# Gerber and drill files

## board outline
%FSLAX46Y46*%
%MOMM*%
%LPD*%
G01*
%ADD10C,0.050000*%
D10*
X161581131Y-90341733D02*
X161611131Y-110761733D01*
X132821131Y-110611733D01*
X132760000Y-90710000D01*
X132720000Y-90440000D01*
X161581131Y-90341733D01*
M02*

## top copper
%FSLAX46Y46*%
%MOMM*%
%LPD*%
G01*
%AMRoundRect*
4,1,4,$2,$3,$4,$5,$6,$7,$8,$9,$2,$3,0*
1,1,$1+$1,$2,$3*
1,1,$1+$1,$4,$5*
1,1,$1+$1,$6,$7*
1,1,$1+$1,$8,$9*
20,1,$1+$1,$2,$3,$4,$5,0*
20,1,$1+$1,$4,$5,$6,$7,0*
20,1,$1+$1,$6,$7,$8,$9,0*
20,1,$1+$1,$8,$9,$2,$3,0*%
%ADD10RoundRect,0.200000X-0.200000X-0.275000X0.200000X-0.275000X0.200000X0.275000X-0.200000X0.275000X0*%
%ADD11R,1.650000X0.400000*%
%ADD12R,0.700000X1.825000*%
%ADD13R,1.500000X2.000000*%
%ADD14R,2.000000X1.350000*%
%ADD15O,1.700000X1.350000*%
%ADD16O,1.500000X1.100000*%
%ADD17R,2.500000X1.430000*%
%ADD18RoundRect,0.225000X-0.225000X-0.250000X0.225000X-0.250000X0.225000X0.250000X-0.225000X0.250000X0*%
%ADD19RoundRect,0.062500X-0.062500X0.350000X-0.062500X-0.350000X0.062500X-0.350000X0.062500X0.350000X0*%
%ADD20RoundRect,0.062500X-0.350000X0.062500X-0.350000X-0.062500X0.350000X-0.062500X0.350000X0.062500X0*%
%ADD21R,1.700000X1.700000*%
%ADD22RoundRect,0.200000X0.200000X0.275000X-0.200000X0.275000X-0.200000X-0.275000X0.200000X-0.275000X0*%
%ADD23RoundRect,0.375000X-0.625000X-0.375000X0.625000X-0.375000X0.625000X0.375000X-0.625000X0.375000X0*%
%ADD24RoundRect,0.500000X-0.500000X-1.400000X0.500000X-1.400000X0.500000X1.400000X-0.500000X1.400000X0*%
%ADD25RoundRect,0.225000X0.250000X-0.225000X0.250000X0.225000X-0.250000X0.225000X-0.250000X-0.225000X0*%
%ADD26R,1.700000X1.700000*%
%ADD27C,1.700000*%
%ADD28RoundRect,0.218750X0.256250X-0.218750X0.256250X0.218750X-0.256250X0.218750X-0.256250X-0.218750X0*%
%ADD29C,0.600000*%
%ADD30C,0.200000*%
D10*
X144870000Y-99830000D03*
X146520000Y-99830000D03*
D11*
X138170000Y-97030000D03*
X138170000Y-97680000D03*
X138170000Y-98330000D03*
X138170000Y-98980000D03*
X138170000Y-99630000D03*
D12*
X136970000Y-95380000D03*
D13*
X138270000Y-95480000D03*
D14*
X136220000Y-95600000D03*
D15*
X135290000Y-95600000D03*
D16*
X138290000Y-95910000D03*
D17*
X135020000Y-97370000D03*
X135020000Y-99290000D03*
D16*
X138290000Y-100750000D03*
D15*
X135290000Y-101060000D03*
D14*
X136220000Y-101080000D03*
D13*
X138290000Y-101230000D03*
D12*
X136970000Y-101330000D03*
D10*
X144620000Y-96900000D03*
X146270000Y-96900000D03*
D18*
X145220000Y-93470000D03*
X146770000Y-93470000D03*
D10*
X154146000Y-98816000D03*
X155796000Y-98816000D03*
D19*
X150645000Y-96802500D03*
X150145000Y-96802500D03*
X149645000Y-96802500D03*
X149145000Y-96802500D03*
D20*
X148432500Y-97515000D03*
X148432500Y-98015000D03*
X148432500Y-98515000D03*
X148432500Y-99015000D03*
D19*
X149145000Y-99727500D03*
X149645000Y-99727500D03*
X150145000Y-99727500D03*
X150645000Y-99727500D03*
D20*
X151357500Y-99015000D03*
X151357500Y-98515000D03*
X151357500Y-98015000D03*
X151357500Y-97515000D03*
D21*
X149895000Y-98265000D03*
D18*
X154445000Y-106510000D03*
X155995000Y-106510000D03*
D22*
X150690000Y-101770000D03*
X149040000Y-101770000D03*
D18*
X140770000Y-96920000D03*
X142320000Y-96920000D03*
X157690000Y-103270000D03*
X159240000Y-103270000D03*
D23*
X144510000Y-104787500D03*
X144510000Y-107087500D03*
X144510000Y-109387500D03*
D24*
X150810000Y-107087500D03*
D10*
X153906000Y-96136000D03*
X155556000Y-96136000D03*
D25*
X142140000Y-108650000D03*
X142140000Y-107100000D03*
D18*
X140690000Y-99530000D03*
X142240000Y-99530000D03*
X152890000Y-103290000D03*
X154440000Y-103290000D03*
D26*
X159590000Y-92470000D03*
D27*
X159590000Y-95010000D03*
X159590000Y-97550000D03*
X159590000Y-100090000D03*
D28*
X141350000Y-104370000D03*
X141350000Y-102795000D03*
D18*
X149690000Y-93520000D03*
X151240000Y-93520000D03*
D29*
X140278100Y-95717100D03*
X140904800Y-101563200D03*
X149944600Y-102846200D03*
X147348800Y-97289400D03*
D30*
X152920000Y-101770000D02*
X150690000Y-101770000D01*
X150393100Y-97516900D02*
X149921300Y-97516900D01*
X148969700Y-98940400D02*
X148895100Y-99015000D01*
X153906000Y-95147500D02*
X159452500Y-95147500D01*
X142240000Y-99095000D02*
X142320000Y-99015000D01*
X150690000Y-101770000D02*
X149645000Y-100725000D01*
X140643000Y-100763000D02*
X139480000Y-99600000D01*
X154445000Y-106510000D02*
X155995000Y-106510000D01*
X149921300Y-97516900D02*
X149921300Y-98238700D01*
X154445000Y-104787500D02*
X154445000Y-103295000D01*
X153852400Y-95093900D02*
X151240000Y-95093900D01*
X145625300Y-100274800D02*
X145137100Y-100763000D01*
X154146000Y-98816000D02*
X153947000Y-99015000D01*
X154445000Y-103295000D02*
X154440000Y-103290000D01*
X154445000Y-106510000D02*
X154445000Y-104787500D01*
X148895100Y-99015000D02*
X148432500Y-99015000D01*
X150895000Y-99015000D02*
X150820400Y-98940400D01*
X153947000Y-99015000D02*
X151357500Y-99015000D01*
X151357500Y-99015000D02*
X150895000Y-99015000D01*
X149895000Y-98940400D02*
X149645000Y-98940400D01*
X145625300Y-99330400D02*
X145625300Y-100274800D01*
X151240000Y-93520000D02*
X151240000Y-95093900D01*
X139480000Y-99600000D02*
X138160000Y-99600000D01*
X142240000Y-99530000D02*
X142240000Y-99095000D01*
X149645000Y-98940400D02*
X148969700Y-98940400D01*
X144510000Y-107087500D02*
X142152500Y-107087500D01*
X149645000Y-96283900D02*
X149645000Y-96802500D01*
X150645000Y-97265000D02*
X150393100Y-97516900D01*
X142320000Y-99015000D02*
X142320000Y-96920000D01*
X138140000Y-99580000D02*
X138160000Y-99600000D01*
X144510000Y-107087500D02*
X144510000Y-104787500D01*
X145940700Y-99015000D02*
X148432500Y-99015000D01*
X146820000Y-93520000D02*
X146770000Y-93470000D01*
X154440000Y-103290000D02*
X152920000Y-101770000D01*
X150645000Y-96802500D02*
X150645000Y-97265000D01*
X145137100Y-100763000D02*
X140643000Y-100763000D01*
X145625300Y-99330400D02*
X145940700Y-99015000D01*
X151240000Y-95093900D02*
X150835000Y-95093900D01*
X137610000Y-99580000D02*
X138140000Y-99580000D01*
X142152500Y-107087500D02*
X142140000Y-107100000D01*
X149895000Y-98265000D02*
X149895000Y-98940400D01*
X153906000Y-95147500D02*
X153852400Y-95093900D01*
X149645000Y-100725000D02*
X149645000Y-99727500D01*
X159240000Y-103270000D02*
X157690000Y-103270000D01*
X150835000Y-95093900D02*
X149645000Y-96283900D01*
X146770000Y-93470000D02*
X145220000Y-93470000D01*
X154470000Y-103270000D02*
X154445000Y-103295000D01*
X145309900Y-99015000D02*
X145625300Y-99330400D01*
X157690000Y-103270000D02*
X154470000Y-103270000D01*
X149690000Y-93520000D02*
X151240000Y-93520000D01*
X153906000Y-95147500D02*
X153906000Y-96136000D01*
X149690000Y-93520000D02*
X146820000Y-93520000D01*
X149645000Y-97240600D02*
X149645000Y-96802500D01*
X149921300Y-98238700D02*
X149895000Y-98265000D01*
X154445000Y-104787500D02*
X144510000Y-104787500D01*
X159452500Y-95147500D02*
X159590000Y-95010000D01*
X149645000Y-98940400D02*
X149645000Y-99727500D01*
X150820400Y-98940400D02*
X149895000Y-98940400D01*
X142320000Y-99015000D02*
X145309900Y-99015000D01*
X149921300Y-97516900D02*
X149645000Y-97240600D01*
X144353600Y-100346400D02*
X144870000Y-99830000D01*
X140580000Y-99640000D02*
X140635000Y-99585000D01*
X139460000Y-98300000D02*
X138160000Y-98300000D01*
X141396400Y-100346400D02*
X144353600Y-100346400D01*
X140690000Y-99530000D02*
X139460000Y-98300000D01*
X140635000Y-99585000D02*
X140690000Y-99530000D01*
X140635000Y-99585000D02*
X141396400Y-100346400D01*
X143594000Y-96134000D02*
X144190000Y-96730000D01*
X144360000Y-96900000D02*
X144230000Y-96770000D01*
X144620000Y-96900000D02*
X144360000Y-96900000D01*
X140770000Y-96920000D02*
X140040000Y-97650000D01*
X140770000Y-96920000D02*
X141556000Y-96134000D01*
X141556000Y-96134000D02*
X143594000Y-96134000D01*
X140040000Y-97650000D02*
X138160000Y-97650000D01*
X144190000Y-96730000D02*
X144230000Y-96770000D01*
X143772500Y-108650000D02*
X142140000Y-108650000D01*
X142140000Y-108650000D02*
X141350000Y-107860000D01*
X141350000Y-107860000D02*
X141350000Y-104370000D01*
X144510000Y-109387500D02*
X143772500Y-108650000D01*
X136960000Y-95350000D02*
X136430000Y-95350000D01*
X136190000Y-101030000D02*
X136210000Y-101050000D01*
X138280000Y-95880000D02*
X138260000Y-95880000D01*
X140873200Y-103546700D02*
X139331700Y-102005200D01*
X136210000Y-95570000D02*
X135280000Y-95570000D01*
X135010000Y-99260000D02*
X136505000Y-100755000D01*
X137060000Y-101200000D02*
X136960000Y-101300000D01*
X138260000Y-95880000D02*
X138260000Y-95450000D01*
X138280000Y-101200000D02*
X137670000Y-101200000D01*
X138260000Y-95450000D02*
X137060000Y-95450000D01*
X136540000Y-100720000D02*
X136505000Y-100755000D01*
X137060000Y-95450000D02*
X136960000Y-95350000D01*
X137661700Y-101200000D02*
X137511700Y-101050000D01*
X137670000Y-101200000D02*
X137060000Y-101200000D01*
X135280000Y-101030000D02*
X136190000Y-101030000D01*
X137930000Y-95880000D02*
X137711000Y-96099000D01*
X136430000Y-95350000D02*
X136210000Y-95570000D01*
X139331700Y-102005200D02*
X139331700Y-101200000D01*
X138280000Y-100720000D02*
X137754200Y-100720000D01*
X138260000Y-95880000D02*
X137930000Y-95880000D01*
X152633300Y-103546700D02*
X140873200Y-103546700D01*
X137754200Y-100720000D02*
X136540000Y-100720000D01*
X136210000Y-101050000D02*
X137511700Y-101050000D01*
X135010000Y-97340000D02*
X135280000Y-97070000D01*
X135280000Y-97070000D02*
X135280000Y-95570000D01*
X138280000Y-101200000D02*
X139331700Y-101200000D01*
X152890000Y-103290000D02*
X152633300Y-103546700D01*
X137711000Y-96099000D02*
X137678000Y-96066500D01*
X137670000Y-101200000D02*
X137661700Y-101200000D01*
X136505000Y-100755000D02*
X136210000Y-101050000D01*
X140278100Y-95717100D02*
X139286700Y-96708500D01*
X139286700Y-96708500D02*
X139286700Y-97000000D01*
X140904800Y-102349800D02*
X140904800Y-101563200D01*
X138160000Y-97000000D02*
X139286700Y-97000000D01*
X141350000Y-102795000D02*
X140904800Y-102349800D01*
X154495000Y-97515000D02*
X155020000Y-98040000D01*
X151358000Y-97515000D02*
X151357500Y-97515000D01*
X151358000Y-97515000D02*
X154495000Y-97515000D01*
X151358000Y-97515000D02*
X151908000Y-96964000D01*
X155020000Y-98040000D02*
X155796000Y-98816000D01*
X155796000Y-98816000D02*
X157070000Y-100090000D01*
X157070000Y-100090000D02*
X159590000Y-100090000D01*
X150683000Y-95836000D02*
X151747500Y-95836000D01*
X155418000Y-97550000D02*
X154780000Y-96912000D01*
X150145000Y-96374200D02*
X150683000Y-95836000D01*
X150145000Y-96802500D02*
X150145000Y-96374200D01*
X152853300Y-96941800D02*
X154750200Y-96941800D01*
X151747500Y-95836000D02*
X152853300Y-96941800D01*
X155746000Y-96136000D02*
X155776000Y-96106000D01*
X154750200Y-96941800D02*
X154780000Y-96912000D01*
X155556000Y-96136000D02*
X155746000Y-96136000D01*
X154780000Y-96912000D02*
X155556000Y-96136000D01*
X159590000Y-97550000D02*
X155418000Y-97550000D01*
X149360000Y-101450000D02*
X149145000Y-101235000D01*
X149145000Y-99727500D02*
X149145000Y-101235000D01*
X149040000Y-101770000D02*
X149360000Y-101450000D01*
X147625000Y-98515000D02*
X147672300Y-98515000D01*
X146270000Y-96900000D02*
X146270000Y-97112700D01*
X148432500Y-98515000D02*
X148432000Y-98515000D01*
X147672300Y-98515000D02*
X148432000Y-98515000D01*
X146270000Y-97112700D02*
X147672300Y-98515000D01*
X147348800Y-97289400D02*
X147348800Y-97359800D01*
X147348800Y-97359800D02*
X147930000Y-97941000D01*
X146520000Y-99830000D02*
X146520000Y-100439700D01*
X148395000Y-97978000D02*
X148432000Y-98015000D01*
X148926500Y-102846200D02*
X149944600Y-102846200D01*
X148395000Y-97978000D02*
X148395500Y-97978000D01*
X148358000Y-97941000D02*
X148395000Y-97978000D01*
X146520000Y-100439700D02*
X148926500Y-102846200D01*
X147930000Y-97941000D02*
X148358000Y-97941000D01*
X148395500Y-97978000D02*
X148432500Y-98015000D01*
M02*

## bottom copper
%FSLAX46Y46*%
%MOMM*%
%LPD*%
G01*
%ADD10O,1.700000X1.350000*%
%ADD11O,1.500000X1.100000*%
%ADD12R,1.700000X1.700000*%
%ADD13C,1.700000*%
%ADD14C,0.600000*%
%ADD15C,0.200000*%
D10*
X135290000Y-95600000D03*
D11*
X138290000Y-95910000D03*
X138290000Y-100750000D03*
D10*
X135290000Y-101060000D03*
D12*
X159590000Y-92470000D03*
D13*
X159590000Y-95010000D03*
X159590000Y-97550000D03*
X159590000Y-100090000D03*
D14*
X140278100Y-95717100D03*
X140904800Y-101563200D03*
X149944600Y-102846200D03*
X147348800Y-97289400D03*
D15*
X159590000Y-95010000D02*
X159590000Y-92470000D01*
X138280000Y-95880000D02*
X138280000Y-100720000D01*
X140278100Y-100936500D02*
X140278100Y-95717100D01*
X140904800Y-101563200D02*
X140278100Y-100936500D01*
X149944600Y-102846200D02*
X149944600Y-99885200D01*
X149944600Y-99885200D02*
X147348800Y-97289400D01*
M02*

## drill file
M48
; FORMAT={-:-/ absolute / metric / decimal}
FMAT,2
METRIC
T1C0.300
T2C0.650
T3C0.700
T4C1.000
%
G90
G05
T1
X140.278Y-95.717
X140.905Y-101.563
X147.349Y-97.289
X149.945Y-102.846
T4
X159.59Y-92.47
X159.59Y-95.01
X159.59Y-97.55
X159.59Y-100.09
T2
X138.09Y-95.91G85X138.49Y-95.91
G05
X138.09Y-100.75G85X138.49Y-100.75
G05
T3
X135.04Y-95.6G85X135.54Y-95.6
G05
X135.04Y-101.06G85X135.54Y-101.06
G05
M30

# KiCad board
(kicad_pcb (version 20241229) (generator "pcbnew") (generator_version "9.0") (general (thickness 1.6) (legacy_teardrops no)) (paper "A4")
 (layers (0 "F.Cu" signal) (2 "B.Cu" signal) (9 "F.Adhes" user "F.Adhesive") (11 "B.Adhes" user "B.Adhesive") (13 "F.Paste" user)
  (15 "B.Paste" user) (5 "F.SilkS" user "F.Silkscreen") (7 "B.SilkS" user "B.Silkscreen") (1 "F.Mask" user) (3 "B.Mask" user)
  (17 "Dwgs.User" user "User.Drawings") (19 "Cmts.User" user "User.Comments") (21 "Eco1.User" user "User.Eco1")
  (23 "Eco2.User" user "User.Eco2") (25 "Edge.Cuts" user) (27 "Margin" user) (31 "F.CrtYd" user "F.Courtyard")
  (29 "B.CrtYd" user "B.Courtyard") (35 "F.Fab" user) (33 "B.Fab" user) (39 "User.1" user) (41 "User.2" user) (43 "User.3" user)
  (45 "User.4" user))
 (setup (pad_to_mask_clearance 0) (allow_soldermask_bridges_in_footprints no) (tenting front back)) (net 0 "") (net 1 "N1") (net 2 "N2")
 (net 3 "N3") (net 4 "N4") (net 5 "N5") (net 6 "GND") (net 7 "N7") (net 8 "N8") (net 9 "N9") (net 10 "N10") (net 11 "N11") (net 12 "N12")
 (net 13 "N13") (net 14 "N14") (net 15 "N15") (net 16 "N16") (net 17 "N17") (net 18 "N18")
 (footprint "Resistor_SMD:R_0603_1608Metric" (layer "F.Cu") (at 145.695 99.83)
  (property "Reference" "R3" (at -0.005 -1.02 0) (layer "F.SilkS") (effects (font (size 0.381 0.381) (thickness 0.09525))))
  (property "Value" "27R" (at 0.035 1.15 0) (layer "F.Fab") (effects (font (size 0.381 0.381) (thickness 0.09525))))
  (pad "1" smd roundrect (at -0.825 0) (size 0.8 0.95) (layers "F.Cu" "F.Mask" "F.Paste") (roundrect_rratio 0.25) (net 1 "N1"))
  (pad "2" smd roundrect (at 0.825 0) (size 0.8 0.95) (layers "F.Cu" "F.Mask" "F.Paste") (roundrect_rratio 0.25) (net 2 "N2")))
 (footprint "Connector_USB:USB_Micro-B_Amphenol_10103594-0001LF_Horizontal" (layer "F.Cu") (at 136.405 98.355 -90)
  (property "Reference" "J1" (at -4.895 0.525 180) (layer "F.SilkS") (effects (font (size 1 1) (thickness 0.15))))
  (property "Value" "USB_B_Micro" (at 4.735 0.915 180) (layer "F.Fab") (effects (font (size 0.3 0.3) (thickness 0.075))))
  (pad "1" smd rect (at -1.325 -1.765) (size 1.65 0.4) (layers "F.Cu" "F.Mask" "F.Paste") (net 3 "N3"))
  (pad "2" smd rect (at -0.675 -1.765) (size 1.65 0.4) (layers "F.Cu" "F.Mask" "F.Paste") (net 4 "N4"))
  (pad "3" smd rect (at -0.025 -1.765) (size 1.65 0.4) (layers "F.Cu" "F.Mask" "F.Paste") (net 1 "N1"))
  (pad "4" smd rect (at 0.625 -1.765) (size 1.65 0.4) (layers "F.Cu" "F.Mask" "F.Paste") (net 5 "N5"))
  (pad "5" smd rect (at 1.275 -1.765) (size 1.65 0.4) (layers "F.Cu" "F.Mask" "F.Paste") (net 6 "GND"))
  (pad "6" smd rect (at -2.975 -0.565 270) (size 1.825 0.7) (layers "F.Cu" "F.Mask" "F.Paste") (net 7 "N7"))
  (pad "6" smd rect (at -2.875 -1.865 270) (size 2 1.5) (layers "F.Cu" "F.Mask" "F.Paste") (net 7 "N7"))
  (pad "6" smd rect (at -2.755 0.185 270) (size 1.35 2) (layers "F.Cu" "F.Mask" "F.Paste") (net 7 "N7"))
  (pad "6" thru_hole oval (at -2.755 1.115) (size 1.7 1.35) (drill oval 1.2 0.7) (layers "*.Cu" "*.Mask") (remove_unused_layers no)
   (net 7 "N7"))
  (pad "6" thru_hole oval (at -2.445 -1.885) (size 1.5 1.1) (drill oval 1.05 0.65) (layers "*.Cu" "*.Mask") (remove_unused_layers no)
   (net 7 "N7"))
  (pad "6" smd rect (at -0.985 1.385) (size 2.5 1.43) (layers "F.Cu" "F.Mask" "F.Paste") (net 7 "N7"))
  (pad "6" smd rect (at 0.935 1.385) (size 2.5 1.43) (layers "F.Cu" "F.Mask" "F.Paste") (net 7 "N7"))
  (pad "6" thru_hole oval (at 2.395 -1.885) (size 1.5 1.1) (drill oval 1.05 0.65) (layers "*.Cu" "*.Mask") (remove_unused_layers no)
   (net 7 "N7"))
  (pad "6" thru_hole oval (at 2.705 1.115) (size 1.7 1.35) (drill oval 1.2 0.7) (layers "*.Cu" "*.Mask") (remove_unused_layers no)
   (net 7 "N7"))
  (pad "6" smd rect (at 2.725 0.185 270) (size 1.35 2) (layers "F.Cu" "F.Mask" "F.Paste") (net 7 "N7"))
  (pad "6" smd rect (at 2.875 -1.885 270) (size 2 1.5) (layers "F.Cu" "F.Mask" "F.Paste") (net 7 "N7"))
  (pad "6" smd rect (at 2.975 -0.565 270) (size 1.825 0.7) (layers "F.Cu" "F.Mask" "F.Paste") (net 7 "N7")))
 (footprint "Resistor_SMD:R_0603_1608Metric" (layer "F.Cu") (at 145.445 96.9)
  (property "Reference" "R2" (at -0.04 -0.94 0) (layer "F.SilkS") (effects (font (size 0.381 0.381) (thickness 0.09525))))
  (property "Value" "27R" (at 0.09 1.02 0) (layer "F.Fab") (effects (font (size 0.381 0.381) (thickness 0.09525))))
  (pad "1" smd roundrect (at -0.825 0) (size 0.8 0.95) (layers "F.Cu" "F.Mask" "F.Paste") (roundrect_rratio 0.25) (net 4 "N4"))
  (pad "2" smd roundrect (at 0.825 0) (size 0.8 0.95) (layers "F.Cu" "F.Mask" "F.Paste") (roundrect_rratio 0.25) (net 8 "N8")))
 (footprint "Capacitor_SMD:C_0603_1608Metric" (layer "F.Cu") (at 145.995 93.47)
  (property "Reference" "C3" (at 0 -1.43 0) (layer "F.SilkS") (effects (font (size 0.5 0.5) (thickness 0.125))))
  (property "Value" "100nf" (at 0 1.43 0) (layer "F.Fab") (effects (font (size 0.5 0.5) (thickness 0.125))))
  (pad "1" smd roundrect (at -0.775 0) (size 0.9 0.95) (layers "F.Cu" "F.Mask" "F.Paste") (roundrect_rratio 0.25) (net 6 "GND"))
  (pad "2" smd roundrect (at 0.775 0) (size 0.9 0.95) (layers "F.Cu" "F.Mask" "F.Paste") (roundrect_rratio 0.25) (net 6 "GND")))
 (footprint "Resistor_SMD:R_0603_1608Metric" (layer "F.Cu") (at 154.971 98.816)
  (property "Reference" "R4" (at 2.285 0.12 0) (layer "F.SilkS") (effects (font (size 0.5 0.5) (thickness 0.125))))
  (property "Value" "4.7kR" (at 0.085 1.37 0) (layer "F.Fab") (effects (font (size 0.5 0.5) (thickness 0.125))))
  (pad "1" smd roundrect (at -0.825 0) (size 0.8 0.95) (layers "F.Cu" "F.Mask" "F.Paste") (roundrect_rratio 0.25) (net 6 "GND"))
  (pad "2" smd roundrect (at 0.825 0) (size 0.8 0.95) (layers "F.Cu" "F.Mask" "F.Paste") (roundrect_rratio 0.25) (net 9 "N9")))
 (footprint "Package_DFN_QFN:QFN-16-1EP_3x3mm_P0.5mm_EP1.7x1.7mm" (layer "F.Cu") (at 149.895 98.265 -90)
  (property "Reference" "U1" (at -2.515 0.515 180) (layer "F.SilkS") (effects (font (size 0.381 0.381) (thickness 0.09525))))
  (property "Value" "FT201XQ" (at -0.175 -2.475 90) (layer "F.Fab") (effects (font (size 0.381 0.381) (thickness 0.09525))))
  (pad "" smd roundrect (at -0.425 -0.425 270) (size 0.69 0.69) (layers "F.Paste") (roundrect_rratio 0.25))
  (pad "" smd roundrect (at -0.425 0.425 270) (size 0.69 0.69) (layers "F.Paste") (roundrect_rratio 0.25))
  (pad "" smd roundrect (at 0.425 -0.425 270) (size 0.69 0.69) (layers "F.Paste") (roundrect_rratio 0.25))
  (pad "" smd roundrect (at 0.425 0.425 270) (size 0.69 0.69) (layers "F.Paste") (roundrect_rratio 0.25))
  (pad "1" smd roundrect (at -1.4625 -0.75 270) (size 0.825 0.25) (layers "F.Cu" "F.Mask" "F.Paste") (roundrect_rratio 0.25) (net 6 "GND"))
  (pad "2" smd roundrect (at -1.4625 -0.25 270) (size 0.825 0.25) (layers "F.Cu" "F.Mask" "F.Paste") (roundrect_rratio 0.25) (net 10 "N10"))
  (pad "3" smd roundrect (at -1.4625 0.25 270) (size 0.825 0.25) (layers "F.Cu" "F.Mask" "F.Paste") (roundrect_rratio 0.25) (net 6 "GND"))
  (pad "4" smd roundrect (at -1.4625 0.75 270) (size 0.825 0.25) (layers "F.Cu" "F.Mask" "F.Paste") (roundrect_rratio 0.25) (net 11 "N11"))
  (pad "5" smd roundrect (at -0.75 1.4625 270) (size 0.25 0.825) (layers "F.Cu" "F.Mask" "F.Paste") (roundrect_rratio 0.25) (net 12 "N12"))
  (pad "6" smd roundrect (at -0.25 1.4625 270) (size 0.25 0.825) (layers "F.Cu" "F.Mask" "F.Paste") (roundrect_rratio 0.25) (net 2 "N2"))
  (pad "7" smd roundrect (at 0.25 1.4625 270) (size 0.25 0.825) (layers "F.Cu" "F.Mask" "F.Paste") (roundrect_rratio 0.25) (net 8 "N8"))
  (pad "8" smd roundrect (at 0.75 1.4625 270) (size 0.25 0.825) (layers "F.Cu" "F.Mask" "F.Paste") (roundrect_rratio 0.25) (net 6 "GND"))
  (pad "9" smd roundrect (at 1.4625 0.75 270) (size 0.825 0.25) (layers "F.Cu" "F.Mask" "F.Paste") (roundrect_rratio 0.25) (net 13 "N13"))
  (pad "10" smd roundrect (at 1.4625 0.25 270) (size 0.825 0.25) (layers "F.Cu" "F.Mask" "F.Paste") (roundrect_rratio 0.25) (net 6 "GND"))
  (pad "11" smd roundrect (at 1.4625 -0.25 270) (size 0.825 0.25) (layers "F.Cu" "F.Mask" "F.Paste") (roundrect_rratio 0.25) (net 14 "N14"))
  (pad "12" smd roundrect (at 1.4625 -0.75 270) (size 0.825 0.25) (layers "F.Cu" "F.Mask" "F.Paste") (roundrect_rratio 0.25) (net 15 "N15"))
  (pad "13" smd roundrect (at 0.75 -1.4625 270) (size 0.25 0.825) (layers "F.Cu" "F.Mask" "F.Paste") (roundrect_rratio 0.25) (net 6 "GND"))
  (pad "14" smd roundrect (at 0.25 -1.4625 270) (size 0.25 0.825) (layers "F.Cu" "F.Mask" "F.Paste") (roundrect_rratio 0.25) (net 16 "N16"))
  (pad "15" smd roundrect (at -0.25 -1.4625 270) (size 0.25 0.825) (layers "F.Cu" "F.Mask" "F.Paste") (roundrect_rratio 0.25) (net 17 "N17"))
  (pad "16" smd roundrect (at -0.75 -1.4625 270) (size 0.25 0.825) (layers "F.Cu" "F.Mask" "F.Paste") (roundrect_rratio 0.25) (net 9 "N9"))
  (pad "17" smd rect (at 0 0 270) (size 1.7 1.7) (layers "F.Cu" "F.Mask") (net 6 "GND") (zone_connect 2)))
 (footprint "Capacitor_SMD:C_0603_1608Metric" (layer "F.Cu") (at 155.22 106.51)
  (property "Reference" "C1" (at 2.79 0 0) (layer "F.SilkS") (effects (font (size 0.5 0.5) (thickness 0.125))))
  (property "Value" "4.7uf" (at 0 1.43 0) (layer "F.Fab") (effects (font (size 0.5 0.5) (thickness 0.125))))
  (pad "1" smd roundrect (at -0.775 0) (size 0.9 0.95) (layers "F.Cu" "F.Mask" "F.Paste") (roundrect_rratio 0.25) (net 6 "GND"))
  (pad "2" smd roundrect (at 0.775 0) (size 0.9 0.95) (layers "F.Cu" "F.Mask" "F.Paste") (roundrect_rratio 0.25) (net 6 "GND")))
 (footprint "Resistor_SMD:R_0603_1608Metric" (layer "F.Cu") (at 149.865 101.77 180)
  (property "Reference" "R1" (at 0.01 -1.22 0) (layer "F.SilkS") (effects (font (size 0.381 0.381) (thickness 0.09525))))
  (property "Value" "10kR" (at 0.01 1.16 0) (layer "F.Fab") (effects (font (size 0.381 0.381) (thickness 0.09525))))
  (pad "1" smd roundrect (at -0.825 0 180) (size 0.8 0.95) (layers "F.Cu" "F.Mask" "F.Paste") (roundrect_rratio 0.25) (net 6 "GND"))
  (pad "2" smd roundrect (at 0.825 0 180) (size 0.8 0.95) (layers "F.Cu" "F.Mask" "F.Paste") (roundrect_rratio 0.25) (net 13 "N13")))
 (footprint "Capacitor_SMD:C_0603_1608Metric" (layer "F.Cu") (at 141.545 96.92)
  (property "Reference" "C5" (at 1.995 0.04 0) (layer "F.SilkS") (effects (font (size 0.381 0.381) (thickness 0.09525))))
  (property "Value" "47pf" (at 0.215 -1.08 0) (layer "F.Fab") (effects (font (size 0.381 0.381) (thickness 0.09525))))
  (pad "1" smd roundrect (at -0.775 0) (size 0.9 0.95) (layers "F.Cu" "F.Mask" "F.Paste") (roundrect_rratio 0.25) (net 4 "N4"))
  (pad "2" smd roundrect (at 0.775 0) (size 0.9 0.95) (layers "F.Cu" "F.Mask" "F.Paste") (roundrect_rratio 0.25) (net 6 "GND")))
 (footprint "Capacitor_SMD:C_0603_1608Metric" (layer "F.Cu") (at 158.465 103.27)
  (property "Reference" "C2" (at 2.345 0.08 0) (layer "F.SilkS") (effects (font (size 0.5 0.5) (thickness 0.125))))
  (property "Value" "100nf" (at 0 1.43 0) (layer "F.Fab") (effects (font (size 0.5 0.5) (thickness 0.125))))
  (pad "1" smd roundrect (at -0.775 0) (size 0.9 0.95) (layers "F.Cu" "F.Mask" "F.Paste") (roundrect_rratio 0.25) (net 6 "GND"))
  (pad "2" smd roundrect (at 0.775 0) (size 0.9 0.95) (layers "F.Cu" "F.Mask" "F.Paste") (roundrect_rratio 0.25) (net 6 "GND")))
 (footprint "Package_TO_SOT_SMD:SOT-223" (layer "F.Cu") (at 147.66 107.0875)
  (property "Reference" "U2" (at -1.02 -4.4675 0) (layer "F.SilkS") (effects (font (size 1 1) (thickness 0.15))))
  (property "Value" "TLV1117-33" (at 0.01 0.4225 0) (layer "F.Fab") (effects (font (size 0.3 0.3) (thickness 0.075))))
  (pad "1" smd roundrect (at -3.15 -2.3) (size 2 1.5) (layers "F.Cu" "F.Mask" "F.Paste") (roundrect_rratio 0.25) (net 6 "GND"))
  (pad "2" smd roundrect (at -3.15 0) (size 2 1.5) (layers "F.Cu" "F.Mask" "F.Paste") (roundrect_rratio 0.25) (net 6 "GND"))
  (pad "3" smd roundrect (at -3.15 2.3) (size 2 1.5) (layers "F.Cu" "F.Mask" "F.Paste") (roundrect_rratio 0.25) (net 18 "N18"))
  (pad "4" smd roundrect (at 3.15 0) (size 2 3.8) (layers "F.Cu" "F.Mask" "F.Paste") (roundrect_rratio 0.25)))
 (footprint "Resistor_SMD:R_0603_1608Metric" (layer "F.Cu") (at 154.731 96.136)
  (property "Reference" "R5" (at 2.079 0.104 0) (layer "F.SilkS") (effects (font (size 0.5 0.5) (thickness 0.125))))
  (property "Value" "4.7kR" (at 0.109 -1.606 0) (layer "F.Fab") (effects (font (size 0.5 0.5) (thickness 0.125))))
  (pad "1" smd roundrect (at -0.825 0) (size 0.8 0.95) (layers "F.Cu" "F.Mask" "F.Paste") (roundrect_rratio 0.25) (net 6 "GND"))
  (pad "2" smd roundrect (at 0.825 0) (size 0.8 0.95) (layers "F.Cu" "F.Mask" "F.Paste") (roundrect_rratio 0.25) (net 10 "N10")))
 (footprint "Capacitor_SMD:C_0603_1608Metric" (layer "F.Cu") (at 142.14 107.875 90)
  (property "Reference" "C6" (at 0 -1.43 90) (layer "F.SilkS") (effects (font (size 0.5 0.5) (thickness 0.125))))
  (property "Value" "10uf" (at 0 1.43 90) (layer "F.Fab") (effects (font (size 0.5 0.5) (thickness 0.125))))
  (pad "1" smd roundrect (at -0.775 0 90) (size 0.9 0.95) (layers "F.Cu" "F.Mask" "F.Paste") (roundrect_rratio 0.25) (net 18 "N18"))
  (pad "2" smd roundrect (at 0.775 0 90) (size 0.9 0.95) (layers "F.Cu" "F.Mask" "F.Paste") (roundrect_rratio 0.25) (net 6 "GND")))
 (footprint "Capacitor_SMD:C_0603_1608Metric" (layer "F.Cu") (at 141.465 99.53)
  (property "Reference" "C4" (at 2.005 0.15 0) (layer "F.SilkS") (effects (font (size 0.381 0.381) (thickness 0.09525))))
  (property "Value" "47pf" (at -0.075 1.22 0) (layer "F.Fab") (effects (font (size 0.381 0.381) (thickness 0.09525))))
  (pad "1" smd roundrect (at -0.775 0) (size 0.9 0.95) (layers "F.Cu" "F.Mask" "F.Paste") (roundrect_rratio 0.25) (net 1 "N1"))
  (pad "2" smd roundrect (at 0.775 0) (size 0.9 0.95) (layers "F.Cu" "F.Mask" "F.Paste") (roundrect_rratio 0.25) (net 6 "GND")))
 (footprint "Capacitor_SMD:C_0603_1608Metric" (layer "F.Cu") (at 153.665 103.29)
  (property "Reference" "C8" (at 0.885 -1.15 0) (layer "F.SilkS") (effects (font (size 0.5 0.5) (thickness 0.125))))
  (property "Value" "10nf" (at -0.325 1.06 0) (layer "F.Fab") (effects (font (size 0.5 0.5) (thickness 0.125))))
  (pad "1" smd roundrect (at -0.775 0) (size 0.9 0.95) (layers "F.Cu" "F.Mask" "F.Paste") (roundrect_rratio 0.25) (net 7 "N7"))
  (pad "2" smd roundrect (at 0.775 0) (size 0.9 0.95) (layers "F.Cu" "F.Mask" "F.Paste") (roundrect_rratio 0.25) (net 6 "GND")))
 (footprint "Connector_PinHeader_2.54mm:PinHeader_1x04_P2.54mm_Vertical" (layer "F.Cu") (at 159.59 92.47)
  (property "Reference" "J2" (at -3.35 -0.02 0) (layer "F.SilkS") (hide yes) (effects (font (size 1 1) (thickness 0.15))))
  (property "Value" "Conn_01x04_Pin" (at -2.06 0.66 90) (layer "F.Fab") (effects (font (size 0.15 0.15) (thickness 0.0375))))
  (pad "1" thru_hole rect (at 0 0) (size 1.7 1.7) (drill 1) (layers "*.Cu" "*.Mask") (remove_unused_layers no) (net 6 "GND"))
  (pad "2" thru_hole circle (at 0 2.54) (size 1.7 1.7) (drill 1) (layers "*.Cu" "*.Mask") (remove_unused_layers no) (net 6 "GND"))
  (pad "3" thru_hole circle (at 0 5.08) (size 1.7 1.7) (drill 1) (layers "*.Cu" "*.Mask") (remove_unused_layers no) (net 10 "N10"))
  (pad "4" thru_hole circle (at 0 7.62) (size 1.7 1.7) (drill 1) (layers "*.Cu" "*.Mask") (remove_unused_layers no) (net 9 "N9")))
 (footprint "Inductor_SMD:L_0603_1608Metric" (layer "F.Cu") (at 141.35 103.5825 90)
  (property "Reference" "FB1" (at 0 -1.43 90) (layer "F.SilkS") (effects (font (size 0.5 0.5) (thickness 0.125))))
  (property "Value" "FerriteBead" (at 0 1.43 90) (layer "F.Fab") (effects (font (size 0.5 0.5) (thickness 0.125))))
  (pad "1" smd roundrect (at -0.7875 0 90) (size 0.875 0.95) (layers "F.Cu" "F.Mask" "F.Paste") (roundrect_rratio 0.25) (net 18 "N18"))
  (pad "2" smd roundrect (at 0.7875 0 90) (size 0.875 0.95) (layers "F.Cu" "F.Mask" "F.Paste") (roundrect_rratio 0.25) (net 3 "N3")))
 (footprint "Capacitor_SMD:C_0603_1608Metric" (layer "F.Cu") (at 150.465 93.52)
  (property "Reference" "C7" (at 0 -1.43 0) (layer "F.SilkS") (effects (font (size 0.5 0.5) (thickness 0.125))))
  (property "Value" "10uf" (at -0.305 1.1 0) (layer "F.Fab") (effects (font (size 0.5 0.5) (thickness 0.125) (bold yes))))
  (pad "1" smd roundrect (at -0.775 0) (size 0.9 0.95) (layers "F.Cu" "F.Mask" "F.Paste") (roundrect_rratio 0.25) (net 6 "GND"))
  (pad "2" smd roundrect (at 0.775 0) (size 0.9 0.95) (layers "F.Cu" "F.Mask" "F.Paste") (roundrect_rratio 0.25) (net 6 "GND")))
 (gr_poly
  (pts (xy 161.581131 90.341733) (xy 161.611131 110.761733) (xy 132.821131 110.611733) (xy 132.76 90.71) (xy 132.72 90.44))
  (stroke (width 0.05) (type solid)) (fill no) (layer "Edge.Cuts"))
 (segment (start 152.92 101.77) (end 150.69 101.77) (width 0.2) (layer "F.Cu") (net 6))
 (segment (start 150.3931 97.5169) (end 149.9213 97.5169) (width 0.2) (layer "F.Cu") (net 6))
 (segment (start 148.9697 98.9404) (end 148.8951 99.015) (width 0.2) (layer "F.Cu") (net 6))
 (segment (start 153.906 95.1475) (end 159.4525 95.1475) (width 0.2) (layer "F.Cu") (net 6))
 (segment (start 142.24 99.095) (end 142.32 99.015) (width 0.2) (layer "F.Cu") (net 6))
 (segment (start 150.69 101.77) (end 149.645 100.725) (width 0.2) (layer "F.Cu") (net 6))
 (segment (start 140.643 100.763) (end 139.48 99.6) (width 0.2) (layer "F.Cu") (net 6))
 (segment (start 154.445 106.51) (end 155.995 106.51) (width 0.2) (layer "F.Cu") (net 6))
 (segment (start 149.9213 97.5169) (end 149.9213 98.2387) (width 0.2) (layer "F.Cu") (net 6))
 (segment (start 154.445 104.7875) (end 154.445 103.295) (width 0.2) (layer "F.Cu") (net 6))
 (segment (start 153.8524 95.0939) (end 151.24 95.0939) (width 0.2) (layer "F.Cu") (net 6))
 (segment (start 145.6253 100.2748) (end 145.1371 100.763) (width 0.2) (layer "F.Cu") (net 6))
 (segment (start 154.146 98.816) (end 153.947 99.015) (width 0.2) (layer "F.Cu") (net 6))
 (segment (start 154.445 103.295) (end 154.44 103.29) (width 0.2) (layer "F.Cu") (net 6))
 (segment (start 154.445 106.51) (end 154.445 104.7875) (width 0.2) (layer "F.Cu") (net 6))
 (segment (start 148.8951 99.015) (end 148.4325 99.015) (width 0.2) (layer "F.Cu") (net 6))
 (segment (start 150.895 99.015) (end 150.8204 98.9404) (width 0.2) (layer "F.Cu") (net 6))
 (segment (start 153.947 99.015) (end 151.3575 99.015) (width 0.2) (layer "F.Cu") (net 6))
 (segment (start 151.3575 99.015) (end 150.895 99.015) (width 0.2) (layer "F.Cu") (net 6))
 (segment (start 149.895 98.9404) (end 149.645 98.9404) (width 0.2) (layer "F.Cu") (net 6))
 (segment (start 145.6253 99.3304) (end 145.6253 100.2748) (width 0.2) (layer "F.Cu") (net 6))
 (segment (start 151.24 93.52) (end 151.24 95.0939) (width 0.2) (layer "F.Cu") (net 6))
 (segment (start 139.48 99.6) (end 138.16 99.6) (width 0.2) (layer "F.Cu") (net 6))
 (segment (start 142.24 99.53) (end 142.24 99.095) (width 0.2) (layer "F.Cu") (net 6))
 (segment (start 149.645 98.9404) (end 148.9697 98.9404) (width 0.2) (layer "F.Cu") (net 6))
 (segment (start 144.51 107.0875) (end 142.1525 107.0875) (width 0.2) (layer "F.Cu") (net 6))
 (segment (start 149.645 96.2839) (end 149.645 96.8025) (width 0.2) (layer "F.Cu") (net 6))
 (segment (start 150.645 97.265) (end 150.3931 97.5169) (width 0.2) (layer "F.Cu") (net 6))
 (segment (start 142.32 99.015) (end 142.32 96.92) (width 0.2) (layer "F.Cu") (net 6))
 (segment (start 138.14 99.58) (end 138.16 99.6) (width 0.2) (layer "F.Cu") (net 6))
 (segment (start 144.51 107.0875) (end 144.51 104.7875) (width 0.2) (layer "F.Cu") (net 6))
 (segment (start 145.9407 99.015) (end 148.4325 99.015) (width 0.2) (layer "F.Cu") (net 6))
 (segment (start 146.82 93.52) (end 146.77 93.47) (width 0.2) (layer "F.Cu") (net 6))
 (segment (start 154.44 103.29) (end 152.92 101.77) (width 0.2) (layer "F.Cu") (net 6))
 (segment (start 150.645 96.8025) (end 150.645 97.265) (width 0.2) (layer "F.Cu") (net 6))
 (segment (start 145.1371 100.763) (end 140.643 100.763) (width 0.2) (layer "F.Cu") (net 6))
 (segment (start 145.6253 99.3304) (end 145.9407 99.015) (width 0.2) (layer "F.Cu") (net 6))
 (segment (start 151.24 95.0939) (end 150.835 95.0939) (width 0.2) (layer "F.Cu") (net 6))
 (segment (start 137.61 99.58) (end 138.14 99.58) (width 0.2) (layer "F.Cu") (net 6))
 (segment (start 142.1525 107.0875) (end 142.14 107.1) (width 0.2) (layer "F.Cu") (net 6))
 (segment (start 149.895 98.265) (end 149.895 98.9404) (width 0.2) (layer "F.Cu") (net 6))
 (segment (start 153.906 95.1475) (end 153.8524 95.0939) (width 0.2) (layer "F.Cu") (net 6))
 (segment (start 149.645 100.725) (end 149.645 99.7275) (width 0.2) (layer "F.Cu") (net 6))
 (segment (start 159.24 103.27) (end 157.69 103.27) (width 0.2) (layer "F.Cu") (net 6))
 (segment (start 150.835 95.0939) (end 149.645 96.2839) (width 0.2) (layer "F.Cu") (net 6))
 (segment (start 146.77 93.47) (end 145.22 93.47) (width 0.2) (layer "F.Cu") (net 6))
 (segment (start 154.47 103.27) (end 154.445 103.295) (width 0.2) (layer "F.Cu") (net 6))
 (segment (start 145.3099 99.015) (end 145.6253 99.3304) (width 0.2) (layer "F.Cu") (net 6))
 (segment (start 157.69 103.27) (end 154.47 103.27) (width 0.2) (layer "F.Cu") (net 6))
 (segment (start 149.69 93.52) (end 151.24 93.52) (width 0.2) (layer "F.Cu") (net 6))
 (segment (start 153.906 95.1475) (end 153.906 96.136) (width 0.2) (layer "F.Cu") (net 6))
 (segment (start 149.69 93.52) (end 146.82 93.52) (width 0.2) (layer "F.Cu") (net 6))
 (segment (start 149.645 97.2406) (end 149.645 96.8025) (width 0.2) (layer "F.Cu") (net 6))
 (segment (start 149.9213 98.2387) (end 149.895 98.265) (width 0.2) (layer "F.Cu") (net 6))
 (segment (start 154.445 104.7875) (end 144.51 104.7875) (width 0.2) (layer "F.Cu") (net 6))
 (segment (start 159.4525 95.1475) (end 159.59 95.01) (width 0.2) (layer "F.Cu") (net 6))
 (segment (start 149.645 98.9404) (end 149.645 99.7275) (width 0.2) (layer "F.Cu") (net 6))
 (segment (start 150.8204 98.9404) (end 149.895 98.9404) (width 0.2) (layer "F.Cu") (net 6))
 (segment (start 142.32 99.015) (end 145.3099 99.015) (width 0.2) (layer "F.Cu") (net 6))
 (segment (start 149.9213 97.5169) (end 149.645 97.2406) (width 0.2) (layer "F.Cu") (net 6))
 (segment (start 159.59 95.01) (end 159.59 92.47) (width 0.2) (layer "B.Cu") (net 6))
 (segment (start 144.3536 100.3464) (end 144.87 99.83) (width 0.2) (layer "F.Cu") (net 1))
 (segment (start 140.58 99.64) (end 140.635 99.585) (width 0.2) (layer "F.Cu") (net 1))
 (segment (start 139.46 98.3) (end 138.16 98.3) (width 0.2) (layer "F.Cu") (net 1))
 (segment (start 141.3964 100.3464) (end 144.3536 100.3464) (width 0.2) (layer "F.Cu") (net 1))
 (segment (start 140.69 99.53) (end 139.46 98.3) (width 0.2) (layer "F.Cu") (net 1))
 (segment (start 140.635 99.585) (end 140.69 99.53) (width 0.2) (layer "F.Cu") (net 1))
 (segment (start 140.635 99.585) (end 141.3964 100.3464) (width 0.2) (layer "F.Cu") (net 1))
 (segment (start 143.594 96.134) (end 144.19 96.73) (width 0.2) (layer "F.Cu") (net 4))
 (segment (start 144.36 96.9) (end 144.23 96.77) (width 0.2) (layer "F.Cu") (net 4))
 (segment (start 144.62 96.9) (end 144.36 96.9) (width 0.2) (layer "F.Cu") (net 4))
 (segment (start 140.77 96.92) (end 140.04 97.65) (width 0.2) (layer "F.Cu") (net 4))
 (segment (start 140.77 96.92) (end 141.556 96.134) (width 0.2) (layer "F.Cu") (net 4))
 (segment (start 141.556 96.134) (end 143.594 96.134) (width 0.2) (layer "F.Cu") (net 4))
 (segment (start 140.04 97.65) (end 138.16 97.65) (width 0.2) (layer "F.Cu") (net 4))
 (segment (start 144.19 96.73) (end 144.23 96.77) (width 0.2) (layer "F.Cu") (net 4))
 (segment (start 143.7725 108.65) (end 142.14 108.65) (width 0.2) (layer "F.Cu") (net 18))
 (segment (start 142.14 108.65) (end 141.35 107.86) (width 0.2) (layer "F.Cu") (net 18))
 (segment (start 141.35 107.86) (end 141.35 104.37) (width 0.2) (layer "F.Cu") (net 18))
 (segment (start 144.51 109.3875) (end 143.7725 108.65) (width 0.2) (layer "F.Cu") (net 18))
 (segment (start 136.96 95.35) (end 136.43 95.35) (width 0.2) (layer "F.Cu") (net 7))
 (segment (start 136.19 101.03) (end 136.21 101.05) (width 0.2) (layer "F.Cu") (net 7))
 (segment (start 138.28 95.88) (end 138.26 95.88) (width 0.2) (layer "F.Cu") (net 7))
 (segment (start 140.8732 103.5467) (end 139.3317 102.0052) (width 0.2) (layer "F.Cu") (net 7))
 (segment (start 136.21 95.57) (end 135.28 95.57) (width 0.2) (layer "F.Cu") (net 7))
 (segment (start 135.01 99.26) (end 136.505 100.755) (width 0.2) (layer "F.Cu") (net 7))
 (segment (start 137.06 101.2) (end 136.96 101.3) (width 0.2) (layer "F.Cu") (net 7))
 (segment (start 138.26 95.88) (end 138.26 95.45) (width 0.2) (layer "F.Cu") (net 7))
 (segment (start 138.28 101.2) (end 137.67 101.2) (width 0.2) (layer "F.Cu") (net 7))
 (segment (start 138.26 95.45) (end 137.06 95.45) (width 0.2) (layer "F.Cu") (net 7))
 (segment (start 136.54 100.72) (end 136.505 100.755) (width 0.2) (layer "F.Cu") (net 7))
 (segment (start 137.06 95.45) (end 136.96 95.35) (width 0.2) (layer "F.Cu") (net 7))
 (segment (start 137.6617 101.2) (end 137.5117 101.05) (width 0.2) (layer "F.Cu") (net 7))
 (segment (start 137.67 101.2) (end 137.06 101.2) (width 0.2) (layer "F.Cu") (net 7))
 (segment (start 135.28 101.03) (end 136.19 101.03) (width 0.2) (layer "F.Cu") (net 7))
 (segment (start 137.93 95.88) (end 137.711 96.099) (width 0.2) (layer "F.Cu") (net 7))
 (segment (start 136.43 95.35) (end 136.21 95.57) (width 0.2) (layer "F.Cu") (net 7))
 (segment (start 139.3317 102.0052) (end 139.3317 101.2) (width 0.2) (layer "F.Cu") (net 7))
 (segment (start 138.28 100.72) (end 137.7542 100.72) (width 0.2) (layer "F.Cu") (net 7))
 (segment (start 138.26 95.88) (end 137.93 95.88) (width 0.2) (layer "F.Cu") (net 7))
 (segment (start 152.6333 103.5467) (end 140.8732 103.5467) (width 0.2) (layer "F.Cu") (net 7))
 (segment (start 137.7542 100.72) (end 136.54 100.72) (width 0.2) (layer "F.Cu") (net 7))
 (segment (start 136.21 101.05) (end 137.5117 101.05) (width 0.2) (layer "F.Cu") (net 7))
 (segment (start 135.01 97.34) (end 135.28 97.07) (width 0.2) (layer "F.Cu") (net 7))
 (segment (start 135.28 97.07) (end 135.28 95.57) (width 0.2) (layer "F.Cu") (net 7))
 (segment (start 138.28 101.2) (end 139.3317 101.2) (width 0.2) (layer "F.Cu") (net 7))
 (segment (start 152.89 103.29) (end 152.6333 103.5467) (width 0.2) (layer "F.Cu") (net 7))
 (segment (start 137.711 96.099) (end 137.678 96.0665) (width 0.2) (layer "F.Cu") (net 7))
 (segment (start 137.67 101.2) (end 137.6617 101.2) (width 0.2) (layer "F.Cu") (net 7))
 (segment (start 136.505 100.755) (end 136.21 101.05) (width 0.2) (layer "F.Cu") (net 7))
 (segment (start 138.28 95.88) (end 138.28 100.72) (width 0.2) (layer "B.Cu") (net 7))
 (segment (start 140.2781 95.7171) (end 139.2867 96.7085) (width 0.2) (layer "F.Cu") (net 3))
 (segment (start 139.2867 96.7085) (end 139.2867 97) (width 0.2) (layer "F.Cu") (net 3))
 (segment (start 140.9048 102.3498) (end 140.9048 101.5632) (width 0.2) (layer "F.Cu") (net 3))
 (segment (start 138.16 97) (end 139.2867 97) (width 0.2) (layer "F.Cu") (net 3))
 (segment (start 141.35 102.795) (end 140.9048 102.3498) (width 0.2) (layer "F.Cu") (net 3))
 (via (at 140.2781 95.7171) (size 0.6) (drill 0.3) (layers "F.Cu" "B.Cu") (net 3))
 (via (at 140.9048 101.5632) (size 0.6) (drill 0.3) (layers "F.Cu" "B.Cu") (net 3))
 (segment (start 140.2781 100.9365) (end 140.2781 95.7171) (width 0.2) (layer "B.Cu") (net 3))
 (segment (start 140.9048 101.5632) (end 140.2781 100.9365) (width 0.2) (layer "B.Cu") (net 3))
 (segment (start 154.495 97.515) (end 155.02 98.04) (width 0.2) (layer "F.Cu") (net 9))
 (segment (start 151.358 97.515) (end 151.3575 97.515) (width 0.2) (layer "F.Cu") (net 9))
 (segment (start 151.358 97.515) (end 154.495 97.515) (width 0.2) (layer "F.Cu") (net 9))
 (segment (start 151.358 97.515) (end 151.908 96.964) (width 0.2) (layer "F.Cu") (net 9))
 (segment (start 155.02 98.04) (end 155.796 98.816) (width 0.2) (layer "F.Cu") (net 9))
 (segment (start 155.796 98.816) (end 157.07 100.09) (width 0.2) (layer "F.Cu") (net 9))
 (segment (start 157.07 100.09) (end 159.59 100.09) (width 0.2) (layer "F.Cu") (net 9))
 (segment (start 150.683 95.836) (end 151.7475 95.836) (width 0.2) (layer "F.Cu") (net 10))
 (segment (start 155.418 97.55) (end 154.78 96.912) (width 0.2) (layer "F.Cu") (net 10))
 (segment (start 150.145 96.3742) (end 150.683 95.836) (width 0.2) (layer "F.Cu") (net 10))
 (segment (start 150.145 96.8025) (end 150.145 96.3742) (width 0.2) (layer "F.Cu") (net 10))
 (segment (start 152.8533 96.9418) (end 154.7502 96.9418) (width 0.2) (layer "F.Cu") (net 10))
 (segment (start 151.7475 95.836) (end 152.8533 96.9418) (width 0.2) (layer "F.Cu") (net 10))
 (segment (start 155.746 96.136) (end 155.776 96.106) (width 0.2) (layer "F.Cu") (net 10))
 (segment (start 154.7502 96.9418) (end 154.78 96.912) (width 0.2) (layer "F.Cu") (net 10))
 (segment (start 155.556 96.136) (end 155.746 96.136) (width 0.2) (layer "F.Cu") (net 10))
 (segment (start 154.78 96.912) (end 155.556 96.136) (width 0.2) (layer "F.Cu") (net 10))
 (segment (start 159.59 97.55) (end 155.418 97.55) (width 0.2) (layer "F.Cu") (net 10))
 (segment (start 149.36 101.45) (end 149.145 101.235) (width 0.2) (layer "F.Cu") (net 13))
 (segment (start 149.145 99.7275) (end 149.145 101.235) (width 0.2) (layer "F.Cu") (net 13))
 (segment (start 149.04 101.77) (end 149.36 101.45) (width 0.2) (layer "F.Cu") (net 13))
 (segment (start 147.625 98.515) (end 147.6723 98.515) (width 0.2) (layer "F.Cu") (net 8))
 (segment (start 146.27 96.9) (end 146.27 97.1127) (width 0.2) (layer "F.Cu") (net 8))
 (segment (start 148.4325 98.515) (end 148.432 98.515) (width 0.2) (layer "F.Cu") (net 8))
 (segment (start 147.6723 98.515) (end 148.432 98.515) (width 0.2) (layer "F.Cu") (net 8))
 (segment (start 146.27 97.1127) (end 147.6723 98.515) (width 0.2) (layer "F.Cu") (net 8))
 (segment (start 147.3488 97.2894) (end 147.3488 97.3598) (width 0.2) (layer "F.Cu") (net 2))
 (segment (start 147.3488 97.3598) (end 147.93 97.941) (width 0.2) (layer "F.Cu") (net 2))
 (segment (start 146.52 99.83) (end 146.52 100.4397) (width 0.2) (layer "F.Cu") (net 2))
 (segment (start 148.395 97.978) (end 148.432 98.015) (width 0.2) (layer "F.Cu") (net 2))
 (segment (start 148.9265 102.8462) (end 149.9446 102.8462) (width 0.2) (layer "F.Cu") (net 2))
 (segment (start 148.395 97.978) (end 148.3955 97.978) (width 0.2) (layer "F.Cu") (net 2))
 (segment (start 148.358 97.941) (end 148.395 97.978) (width 0.2) (layer "F.Cu") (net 2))
 (segment (start 146.52 100.4397) (end 148.9265 102.8462) (width 0.2) (layer "F.Cu") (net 2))
 (segment (start 147.93 97.941) (end 148.358 97.941) (width 0.2) (layer "F.Cu") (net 2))
 (segment (start 148.3955 97.978) (end 148.4325 98.015) (width 0.2) (layer "F.Cu") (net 2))
 (via (at 149.9446 102.8462) (size 0.6) (drill 0.3) (layers "F.Cu" "B.Cu") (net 2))
 (via (at 147.3488 97.2894) (size 0.6) (drill 0.3) (layers "F.Cu" "B.Cu") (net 2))
 (segment (start 149.9446 102.8462) (end 149.9446 99.8852) (width 0.2) (layer "B.Cu") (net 2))
 (segment (start 149.9446 99.8852) (end 147.3488 97.2894) (width 0.2) (layer "B.Cu") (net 2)))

